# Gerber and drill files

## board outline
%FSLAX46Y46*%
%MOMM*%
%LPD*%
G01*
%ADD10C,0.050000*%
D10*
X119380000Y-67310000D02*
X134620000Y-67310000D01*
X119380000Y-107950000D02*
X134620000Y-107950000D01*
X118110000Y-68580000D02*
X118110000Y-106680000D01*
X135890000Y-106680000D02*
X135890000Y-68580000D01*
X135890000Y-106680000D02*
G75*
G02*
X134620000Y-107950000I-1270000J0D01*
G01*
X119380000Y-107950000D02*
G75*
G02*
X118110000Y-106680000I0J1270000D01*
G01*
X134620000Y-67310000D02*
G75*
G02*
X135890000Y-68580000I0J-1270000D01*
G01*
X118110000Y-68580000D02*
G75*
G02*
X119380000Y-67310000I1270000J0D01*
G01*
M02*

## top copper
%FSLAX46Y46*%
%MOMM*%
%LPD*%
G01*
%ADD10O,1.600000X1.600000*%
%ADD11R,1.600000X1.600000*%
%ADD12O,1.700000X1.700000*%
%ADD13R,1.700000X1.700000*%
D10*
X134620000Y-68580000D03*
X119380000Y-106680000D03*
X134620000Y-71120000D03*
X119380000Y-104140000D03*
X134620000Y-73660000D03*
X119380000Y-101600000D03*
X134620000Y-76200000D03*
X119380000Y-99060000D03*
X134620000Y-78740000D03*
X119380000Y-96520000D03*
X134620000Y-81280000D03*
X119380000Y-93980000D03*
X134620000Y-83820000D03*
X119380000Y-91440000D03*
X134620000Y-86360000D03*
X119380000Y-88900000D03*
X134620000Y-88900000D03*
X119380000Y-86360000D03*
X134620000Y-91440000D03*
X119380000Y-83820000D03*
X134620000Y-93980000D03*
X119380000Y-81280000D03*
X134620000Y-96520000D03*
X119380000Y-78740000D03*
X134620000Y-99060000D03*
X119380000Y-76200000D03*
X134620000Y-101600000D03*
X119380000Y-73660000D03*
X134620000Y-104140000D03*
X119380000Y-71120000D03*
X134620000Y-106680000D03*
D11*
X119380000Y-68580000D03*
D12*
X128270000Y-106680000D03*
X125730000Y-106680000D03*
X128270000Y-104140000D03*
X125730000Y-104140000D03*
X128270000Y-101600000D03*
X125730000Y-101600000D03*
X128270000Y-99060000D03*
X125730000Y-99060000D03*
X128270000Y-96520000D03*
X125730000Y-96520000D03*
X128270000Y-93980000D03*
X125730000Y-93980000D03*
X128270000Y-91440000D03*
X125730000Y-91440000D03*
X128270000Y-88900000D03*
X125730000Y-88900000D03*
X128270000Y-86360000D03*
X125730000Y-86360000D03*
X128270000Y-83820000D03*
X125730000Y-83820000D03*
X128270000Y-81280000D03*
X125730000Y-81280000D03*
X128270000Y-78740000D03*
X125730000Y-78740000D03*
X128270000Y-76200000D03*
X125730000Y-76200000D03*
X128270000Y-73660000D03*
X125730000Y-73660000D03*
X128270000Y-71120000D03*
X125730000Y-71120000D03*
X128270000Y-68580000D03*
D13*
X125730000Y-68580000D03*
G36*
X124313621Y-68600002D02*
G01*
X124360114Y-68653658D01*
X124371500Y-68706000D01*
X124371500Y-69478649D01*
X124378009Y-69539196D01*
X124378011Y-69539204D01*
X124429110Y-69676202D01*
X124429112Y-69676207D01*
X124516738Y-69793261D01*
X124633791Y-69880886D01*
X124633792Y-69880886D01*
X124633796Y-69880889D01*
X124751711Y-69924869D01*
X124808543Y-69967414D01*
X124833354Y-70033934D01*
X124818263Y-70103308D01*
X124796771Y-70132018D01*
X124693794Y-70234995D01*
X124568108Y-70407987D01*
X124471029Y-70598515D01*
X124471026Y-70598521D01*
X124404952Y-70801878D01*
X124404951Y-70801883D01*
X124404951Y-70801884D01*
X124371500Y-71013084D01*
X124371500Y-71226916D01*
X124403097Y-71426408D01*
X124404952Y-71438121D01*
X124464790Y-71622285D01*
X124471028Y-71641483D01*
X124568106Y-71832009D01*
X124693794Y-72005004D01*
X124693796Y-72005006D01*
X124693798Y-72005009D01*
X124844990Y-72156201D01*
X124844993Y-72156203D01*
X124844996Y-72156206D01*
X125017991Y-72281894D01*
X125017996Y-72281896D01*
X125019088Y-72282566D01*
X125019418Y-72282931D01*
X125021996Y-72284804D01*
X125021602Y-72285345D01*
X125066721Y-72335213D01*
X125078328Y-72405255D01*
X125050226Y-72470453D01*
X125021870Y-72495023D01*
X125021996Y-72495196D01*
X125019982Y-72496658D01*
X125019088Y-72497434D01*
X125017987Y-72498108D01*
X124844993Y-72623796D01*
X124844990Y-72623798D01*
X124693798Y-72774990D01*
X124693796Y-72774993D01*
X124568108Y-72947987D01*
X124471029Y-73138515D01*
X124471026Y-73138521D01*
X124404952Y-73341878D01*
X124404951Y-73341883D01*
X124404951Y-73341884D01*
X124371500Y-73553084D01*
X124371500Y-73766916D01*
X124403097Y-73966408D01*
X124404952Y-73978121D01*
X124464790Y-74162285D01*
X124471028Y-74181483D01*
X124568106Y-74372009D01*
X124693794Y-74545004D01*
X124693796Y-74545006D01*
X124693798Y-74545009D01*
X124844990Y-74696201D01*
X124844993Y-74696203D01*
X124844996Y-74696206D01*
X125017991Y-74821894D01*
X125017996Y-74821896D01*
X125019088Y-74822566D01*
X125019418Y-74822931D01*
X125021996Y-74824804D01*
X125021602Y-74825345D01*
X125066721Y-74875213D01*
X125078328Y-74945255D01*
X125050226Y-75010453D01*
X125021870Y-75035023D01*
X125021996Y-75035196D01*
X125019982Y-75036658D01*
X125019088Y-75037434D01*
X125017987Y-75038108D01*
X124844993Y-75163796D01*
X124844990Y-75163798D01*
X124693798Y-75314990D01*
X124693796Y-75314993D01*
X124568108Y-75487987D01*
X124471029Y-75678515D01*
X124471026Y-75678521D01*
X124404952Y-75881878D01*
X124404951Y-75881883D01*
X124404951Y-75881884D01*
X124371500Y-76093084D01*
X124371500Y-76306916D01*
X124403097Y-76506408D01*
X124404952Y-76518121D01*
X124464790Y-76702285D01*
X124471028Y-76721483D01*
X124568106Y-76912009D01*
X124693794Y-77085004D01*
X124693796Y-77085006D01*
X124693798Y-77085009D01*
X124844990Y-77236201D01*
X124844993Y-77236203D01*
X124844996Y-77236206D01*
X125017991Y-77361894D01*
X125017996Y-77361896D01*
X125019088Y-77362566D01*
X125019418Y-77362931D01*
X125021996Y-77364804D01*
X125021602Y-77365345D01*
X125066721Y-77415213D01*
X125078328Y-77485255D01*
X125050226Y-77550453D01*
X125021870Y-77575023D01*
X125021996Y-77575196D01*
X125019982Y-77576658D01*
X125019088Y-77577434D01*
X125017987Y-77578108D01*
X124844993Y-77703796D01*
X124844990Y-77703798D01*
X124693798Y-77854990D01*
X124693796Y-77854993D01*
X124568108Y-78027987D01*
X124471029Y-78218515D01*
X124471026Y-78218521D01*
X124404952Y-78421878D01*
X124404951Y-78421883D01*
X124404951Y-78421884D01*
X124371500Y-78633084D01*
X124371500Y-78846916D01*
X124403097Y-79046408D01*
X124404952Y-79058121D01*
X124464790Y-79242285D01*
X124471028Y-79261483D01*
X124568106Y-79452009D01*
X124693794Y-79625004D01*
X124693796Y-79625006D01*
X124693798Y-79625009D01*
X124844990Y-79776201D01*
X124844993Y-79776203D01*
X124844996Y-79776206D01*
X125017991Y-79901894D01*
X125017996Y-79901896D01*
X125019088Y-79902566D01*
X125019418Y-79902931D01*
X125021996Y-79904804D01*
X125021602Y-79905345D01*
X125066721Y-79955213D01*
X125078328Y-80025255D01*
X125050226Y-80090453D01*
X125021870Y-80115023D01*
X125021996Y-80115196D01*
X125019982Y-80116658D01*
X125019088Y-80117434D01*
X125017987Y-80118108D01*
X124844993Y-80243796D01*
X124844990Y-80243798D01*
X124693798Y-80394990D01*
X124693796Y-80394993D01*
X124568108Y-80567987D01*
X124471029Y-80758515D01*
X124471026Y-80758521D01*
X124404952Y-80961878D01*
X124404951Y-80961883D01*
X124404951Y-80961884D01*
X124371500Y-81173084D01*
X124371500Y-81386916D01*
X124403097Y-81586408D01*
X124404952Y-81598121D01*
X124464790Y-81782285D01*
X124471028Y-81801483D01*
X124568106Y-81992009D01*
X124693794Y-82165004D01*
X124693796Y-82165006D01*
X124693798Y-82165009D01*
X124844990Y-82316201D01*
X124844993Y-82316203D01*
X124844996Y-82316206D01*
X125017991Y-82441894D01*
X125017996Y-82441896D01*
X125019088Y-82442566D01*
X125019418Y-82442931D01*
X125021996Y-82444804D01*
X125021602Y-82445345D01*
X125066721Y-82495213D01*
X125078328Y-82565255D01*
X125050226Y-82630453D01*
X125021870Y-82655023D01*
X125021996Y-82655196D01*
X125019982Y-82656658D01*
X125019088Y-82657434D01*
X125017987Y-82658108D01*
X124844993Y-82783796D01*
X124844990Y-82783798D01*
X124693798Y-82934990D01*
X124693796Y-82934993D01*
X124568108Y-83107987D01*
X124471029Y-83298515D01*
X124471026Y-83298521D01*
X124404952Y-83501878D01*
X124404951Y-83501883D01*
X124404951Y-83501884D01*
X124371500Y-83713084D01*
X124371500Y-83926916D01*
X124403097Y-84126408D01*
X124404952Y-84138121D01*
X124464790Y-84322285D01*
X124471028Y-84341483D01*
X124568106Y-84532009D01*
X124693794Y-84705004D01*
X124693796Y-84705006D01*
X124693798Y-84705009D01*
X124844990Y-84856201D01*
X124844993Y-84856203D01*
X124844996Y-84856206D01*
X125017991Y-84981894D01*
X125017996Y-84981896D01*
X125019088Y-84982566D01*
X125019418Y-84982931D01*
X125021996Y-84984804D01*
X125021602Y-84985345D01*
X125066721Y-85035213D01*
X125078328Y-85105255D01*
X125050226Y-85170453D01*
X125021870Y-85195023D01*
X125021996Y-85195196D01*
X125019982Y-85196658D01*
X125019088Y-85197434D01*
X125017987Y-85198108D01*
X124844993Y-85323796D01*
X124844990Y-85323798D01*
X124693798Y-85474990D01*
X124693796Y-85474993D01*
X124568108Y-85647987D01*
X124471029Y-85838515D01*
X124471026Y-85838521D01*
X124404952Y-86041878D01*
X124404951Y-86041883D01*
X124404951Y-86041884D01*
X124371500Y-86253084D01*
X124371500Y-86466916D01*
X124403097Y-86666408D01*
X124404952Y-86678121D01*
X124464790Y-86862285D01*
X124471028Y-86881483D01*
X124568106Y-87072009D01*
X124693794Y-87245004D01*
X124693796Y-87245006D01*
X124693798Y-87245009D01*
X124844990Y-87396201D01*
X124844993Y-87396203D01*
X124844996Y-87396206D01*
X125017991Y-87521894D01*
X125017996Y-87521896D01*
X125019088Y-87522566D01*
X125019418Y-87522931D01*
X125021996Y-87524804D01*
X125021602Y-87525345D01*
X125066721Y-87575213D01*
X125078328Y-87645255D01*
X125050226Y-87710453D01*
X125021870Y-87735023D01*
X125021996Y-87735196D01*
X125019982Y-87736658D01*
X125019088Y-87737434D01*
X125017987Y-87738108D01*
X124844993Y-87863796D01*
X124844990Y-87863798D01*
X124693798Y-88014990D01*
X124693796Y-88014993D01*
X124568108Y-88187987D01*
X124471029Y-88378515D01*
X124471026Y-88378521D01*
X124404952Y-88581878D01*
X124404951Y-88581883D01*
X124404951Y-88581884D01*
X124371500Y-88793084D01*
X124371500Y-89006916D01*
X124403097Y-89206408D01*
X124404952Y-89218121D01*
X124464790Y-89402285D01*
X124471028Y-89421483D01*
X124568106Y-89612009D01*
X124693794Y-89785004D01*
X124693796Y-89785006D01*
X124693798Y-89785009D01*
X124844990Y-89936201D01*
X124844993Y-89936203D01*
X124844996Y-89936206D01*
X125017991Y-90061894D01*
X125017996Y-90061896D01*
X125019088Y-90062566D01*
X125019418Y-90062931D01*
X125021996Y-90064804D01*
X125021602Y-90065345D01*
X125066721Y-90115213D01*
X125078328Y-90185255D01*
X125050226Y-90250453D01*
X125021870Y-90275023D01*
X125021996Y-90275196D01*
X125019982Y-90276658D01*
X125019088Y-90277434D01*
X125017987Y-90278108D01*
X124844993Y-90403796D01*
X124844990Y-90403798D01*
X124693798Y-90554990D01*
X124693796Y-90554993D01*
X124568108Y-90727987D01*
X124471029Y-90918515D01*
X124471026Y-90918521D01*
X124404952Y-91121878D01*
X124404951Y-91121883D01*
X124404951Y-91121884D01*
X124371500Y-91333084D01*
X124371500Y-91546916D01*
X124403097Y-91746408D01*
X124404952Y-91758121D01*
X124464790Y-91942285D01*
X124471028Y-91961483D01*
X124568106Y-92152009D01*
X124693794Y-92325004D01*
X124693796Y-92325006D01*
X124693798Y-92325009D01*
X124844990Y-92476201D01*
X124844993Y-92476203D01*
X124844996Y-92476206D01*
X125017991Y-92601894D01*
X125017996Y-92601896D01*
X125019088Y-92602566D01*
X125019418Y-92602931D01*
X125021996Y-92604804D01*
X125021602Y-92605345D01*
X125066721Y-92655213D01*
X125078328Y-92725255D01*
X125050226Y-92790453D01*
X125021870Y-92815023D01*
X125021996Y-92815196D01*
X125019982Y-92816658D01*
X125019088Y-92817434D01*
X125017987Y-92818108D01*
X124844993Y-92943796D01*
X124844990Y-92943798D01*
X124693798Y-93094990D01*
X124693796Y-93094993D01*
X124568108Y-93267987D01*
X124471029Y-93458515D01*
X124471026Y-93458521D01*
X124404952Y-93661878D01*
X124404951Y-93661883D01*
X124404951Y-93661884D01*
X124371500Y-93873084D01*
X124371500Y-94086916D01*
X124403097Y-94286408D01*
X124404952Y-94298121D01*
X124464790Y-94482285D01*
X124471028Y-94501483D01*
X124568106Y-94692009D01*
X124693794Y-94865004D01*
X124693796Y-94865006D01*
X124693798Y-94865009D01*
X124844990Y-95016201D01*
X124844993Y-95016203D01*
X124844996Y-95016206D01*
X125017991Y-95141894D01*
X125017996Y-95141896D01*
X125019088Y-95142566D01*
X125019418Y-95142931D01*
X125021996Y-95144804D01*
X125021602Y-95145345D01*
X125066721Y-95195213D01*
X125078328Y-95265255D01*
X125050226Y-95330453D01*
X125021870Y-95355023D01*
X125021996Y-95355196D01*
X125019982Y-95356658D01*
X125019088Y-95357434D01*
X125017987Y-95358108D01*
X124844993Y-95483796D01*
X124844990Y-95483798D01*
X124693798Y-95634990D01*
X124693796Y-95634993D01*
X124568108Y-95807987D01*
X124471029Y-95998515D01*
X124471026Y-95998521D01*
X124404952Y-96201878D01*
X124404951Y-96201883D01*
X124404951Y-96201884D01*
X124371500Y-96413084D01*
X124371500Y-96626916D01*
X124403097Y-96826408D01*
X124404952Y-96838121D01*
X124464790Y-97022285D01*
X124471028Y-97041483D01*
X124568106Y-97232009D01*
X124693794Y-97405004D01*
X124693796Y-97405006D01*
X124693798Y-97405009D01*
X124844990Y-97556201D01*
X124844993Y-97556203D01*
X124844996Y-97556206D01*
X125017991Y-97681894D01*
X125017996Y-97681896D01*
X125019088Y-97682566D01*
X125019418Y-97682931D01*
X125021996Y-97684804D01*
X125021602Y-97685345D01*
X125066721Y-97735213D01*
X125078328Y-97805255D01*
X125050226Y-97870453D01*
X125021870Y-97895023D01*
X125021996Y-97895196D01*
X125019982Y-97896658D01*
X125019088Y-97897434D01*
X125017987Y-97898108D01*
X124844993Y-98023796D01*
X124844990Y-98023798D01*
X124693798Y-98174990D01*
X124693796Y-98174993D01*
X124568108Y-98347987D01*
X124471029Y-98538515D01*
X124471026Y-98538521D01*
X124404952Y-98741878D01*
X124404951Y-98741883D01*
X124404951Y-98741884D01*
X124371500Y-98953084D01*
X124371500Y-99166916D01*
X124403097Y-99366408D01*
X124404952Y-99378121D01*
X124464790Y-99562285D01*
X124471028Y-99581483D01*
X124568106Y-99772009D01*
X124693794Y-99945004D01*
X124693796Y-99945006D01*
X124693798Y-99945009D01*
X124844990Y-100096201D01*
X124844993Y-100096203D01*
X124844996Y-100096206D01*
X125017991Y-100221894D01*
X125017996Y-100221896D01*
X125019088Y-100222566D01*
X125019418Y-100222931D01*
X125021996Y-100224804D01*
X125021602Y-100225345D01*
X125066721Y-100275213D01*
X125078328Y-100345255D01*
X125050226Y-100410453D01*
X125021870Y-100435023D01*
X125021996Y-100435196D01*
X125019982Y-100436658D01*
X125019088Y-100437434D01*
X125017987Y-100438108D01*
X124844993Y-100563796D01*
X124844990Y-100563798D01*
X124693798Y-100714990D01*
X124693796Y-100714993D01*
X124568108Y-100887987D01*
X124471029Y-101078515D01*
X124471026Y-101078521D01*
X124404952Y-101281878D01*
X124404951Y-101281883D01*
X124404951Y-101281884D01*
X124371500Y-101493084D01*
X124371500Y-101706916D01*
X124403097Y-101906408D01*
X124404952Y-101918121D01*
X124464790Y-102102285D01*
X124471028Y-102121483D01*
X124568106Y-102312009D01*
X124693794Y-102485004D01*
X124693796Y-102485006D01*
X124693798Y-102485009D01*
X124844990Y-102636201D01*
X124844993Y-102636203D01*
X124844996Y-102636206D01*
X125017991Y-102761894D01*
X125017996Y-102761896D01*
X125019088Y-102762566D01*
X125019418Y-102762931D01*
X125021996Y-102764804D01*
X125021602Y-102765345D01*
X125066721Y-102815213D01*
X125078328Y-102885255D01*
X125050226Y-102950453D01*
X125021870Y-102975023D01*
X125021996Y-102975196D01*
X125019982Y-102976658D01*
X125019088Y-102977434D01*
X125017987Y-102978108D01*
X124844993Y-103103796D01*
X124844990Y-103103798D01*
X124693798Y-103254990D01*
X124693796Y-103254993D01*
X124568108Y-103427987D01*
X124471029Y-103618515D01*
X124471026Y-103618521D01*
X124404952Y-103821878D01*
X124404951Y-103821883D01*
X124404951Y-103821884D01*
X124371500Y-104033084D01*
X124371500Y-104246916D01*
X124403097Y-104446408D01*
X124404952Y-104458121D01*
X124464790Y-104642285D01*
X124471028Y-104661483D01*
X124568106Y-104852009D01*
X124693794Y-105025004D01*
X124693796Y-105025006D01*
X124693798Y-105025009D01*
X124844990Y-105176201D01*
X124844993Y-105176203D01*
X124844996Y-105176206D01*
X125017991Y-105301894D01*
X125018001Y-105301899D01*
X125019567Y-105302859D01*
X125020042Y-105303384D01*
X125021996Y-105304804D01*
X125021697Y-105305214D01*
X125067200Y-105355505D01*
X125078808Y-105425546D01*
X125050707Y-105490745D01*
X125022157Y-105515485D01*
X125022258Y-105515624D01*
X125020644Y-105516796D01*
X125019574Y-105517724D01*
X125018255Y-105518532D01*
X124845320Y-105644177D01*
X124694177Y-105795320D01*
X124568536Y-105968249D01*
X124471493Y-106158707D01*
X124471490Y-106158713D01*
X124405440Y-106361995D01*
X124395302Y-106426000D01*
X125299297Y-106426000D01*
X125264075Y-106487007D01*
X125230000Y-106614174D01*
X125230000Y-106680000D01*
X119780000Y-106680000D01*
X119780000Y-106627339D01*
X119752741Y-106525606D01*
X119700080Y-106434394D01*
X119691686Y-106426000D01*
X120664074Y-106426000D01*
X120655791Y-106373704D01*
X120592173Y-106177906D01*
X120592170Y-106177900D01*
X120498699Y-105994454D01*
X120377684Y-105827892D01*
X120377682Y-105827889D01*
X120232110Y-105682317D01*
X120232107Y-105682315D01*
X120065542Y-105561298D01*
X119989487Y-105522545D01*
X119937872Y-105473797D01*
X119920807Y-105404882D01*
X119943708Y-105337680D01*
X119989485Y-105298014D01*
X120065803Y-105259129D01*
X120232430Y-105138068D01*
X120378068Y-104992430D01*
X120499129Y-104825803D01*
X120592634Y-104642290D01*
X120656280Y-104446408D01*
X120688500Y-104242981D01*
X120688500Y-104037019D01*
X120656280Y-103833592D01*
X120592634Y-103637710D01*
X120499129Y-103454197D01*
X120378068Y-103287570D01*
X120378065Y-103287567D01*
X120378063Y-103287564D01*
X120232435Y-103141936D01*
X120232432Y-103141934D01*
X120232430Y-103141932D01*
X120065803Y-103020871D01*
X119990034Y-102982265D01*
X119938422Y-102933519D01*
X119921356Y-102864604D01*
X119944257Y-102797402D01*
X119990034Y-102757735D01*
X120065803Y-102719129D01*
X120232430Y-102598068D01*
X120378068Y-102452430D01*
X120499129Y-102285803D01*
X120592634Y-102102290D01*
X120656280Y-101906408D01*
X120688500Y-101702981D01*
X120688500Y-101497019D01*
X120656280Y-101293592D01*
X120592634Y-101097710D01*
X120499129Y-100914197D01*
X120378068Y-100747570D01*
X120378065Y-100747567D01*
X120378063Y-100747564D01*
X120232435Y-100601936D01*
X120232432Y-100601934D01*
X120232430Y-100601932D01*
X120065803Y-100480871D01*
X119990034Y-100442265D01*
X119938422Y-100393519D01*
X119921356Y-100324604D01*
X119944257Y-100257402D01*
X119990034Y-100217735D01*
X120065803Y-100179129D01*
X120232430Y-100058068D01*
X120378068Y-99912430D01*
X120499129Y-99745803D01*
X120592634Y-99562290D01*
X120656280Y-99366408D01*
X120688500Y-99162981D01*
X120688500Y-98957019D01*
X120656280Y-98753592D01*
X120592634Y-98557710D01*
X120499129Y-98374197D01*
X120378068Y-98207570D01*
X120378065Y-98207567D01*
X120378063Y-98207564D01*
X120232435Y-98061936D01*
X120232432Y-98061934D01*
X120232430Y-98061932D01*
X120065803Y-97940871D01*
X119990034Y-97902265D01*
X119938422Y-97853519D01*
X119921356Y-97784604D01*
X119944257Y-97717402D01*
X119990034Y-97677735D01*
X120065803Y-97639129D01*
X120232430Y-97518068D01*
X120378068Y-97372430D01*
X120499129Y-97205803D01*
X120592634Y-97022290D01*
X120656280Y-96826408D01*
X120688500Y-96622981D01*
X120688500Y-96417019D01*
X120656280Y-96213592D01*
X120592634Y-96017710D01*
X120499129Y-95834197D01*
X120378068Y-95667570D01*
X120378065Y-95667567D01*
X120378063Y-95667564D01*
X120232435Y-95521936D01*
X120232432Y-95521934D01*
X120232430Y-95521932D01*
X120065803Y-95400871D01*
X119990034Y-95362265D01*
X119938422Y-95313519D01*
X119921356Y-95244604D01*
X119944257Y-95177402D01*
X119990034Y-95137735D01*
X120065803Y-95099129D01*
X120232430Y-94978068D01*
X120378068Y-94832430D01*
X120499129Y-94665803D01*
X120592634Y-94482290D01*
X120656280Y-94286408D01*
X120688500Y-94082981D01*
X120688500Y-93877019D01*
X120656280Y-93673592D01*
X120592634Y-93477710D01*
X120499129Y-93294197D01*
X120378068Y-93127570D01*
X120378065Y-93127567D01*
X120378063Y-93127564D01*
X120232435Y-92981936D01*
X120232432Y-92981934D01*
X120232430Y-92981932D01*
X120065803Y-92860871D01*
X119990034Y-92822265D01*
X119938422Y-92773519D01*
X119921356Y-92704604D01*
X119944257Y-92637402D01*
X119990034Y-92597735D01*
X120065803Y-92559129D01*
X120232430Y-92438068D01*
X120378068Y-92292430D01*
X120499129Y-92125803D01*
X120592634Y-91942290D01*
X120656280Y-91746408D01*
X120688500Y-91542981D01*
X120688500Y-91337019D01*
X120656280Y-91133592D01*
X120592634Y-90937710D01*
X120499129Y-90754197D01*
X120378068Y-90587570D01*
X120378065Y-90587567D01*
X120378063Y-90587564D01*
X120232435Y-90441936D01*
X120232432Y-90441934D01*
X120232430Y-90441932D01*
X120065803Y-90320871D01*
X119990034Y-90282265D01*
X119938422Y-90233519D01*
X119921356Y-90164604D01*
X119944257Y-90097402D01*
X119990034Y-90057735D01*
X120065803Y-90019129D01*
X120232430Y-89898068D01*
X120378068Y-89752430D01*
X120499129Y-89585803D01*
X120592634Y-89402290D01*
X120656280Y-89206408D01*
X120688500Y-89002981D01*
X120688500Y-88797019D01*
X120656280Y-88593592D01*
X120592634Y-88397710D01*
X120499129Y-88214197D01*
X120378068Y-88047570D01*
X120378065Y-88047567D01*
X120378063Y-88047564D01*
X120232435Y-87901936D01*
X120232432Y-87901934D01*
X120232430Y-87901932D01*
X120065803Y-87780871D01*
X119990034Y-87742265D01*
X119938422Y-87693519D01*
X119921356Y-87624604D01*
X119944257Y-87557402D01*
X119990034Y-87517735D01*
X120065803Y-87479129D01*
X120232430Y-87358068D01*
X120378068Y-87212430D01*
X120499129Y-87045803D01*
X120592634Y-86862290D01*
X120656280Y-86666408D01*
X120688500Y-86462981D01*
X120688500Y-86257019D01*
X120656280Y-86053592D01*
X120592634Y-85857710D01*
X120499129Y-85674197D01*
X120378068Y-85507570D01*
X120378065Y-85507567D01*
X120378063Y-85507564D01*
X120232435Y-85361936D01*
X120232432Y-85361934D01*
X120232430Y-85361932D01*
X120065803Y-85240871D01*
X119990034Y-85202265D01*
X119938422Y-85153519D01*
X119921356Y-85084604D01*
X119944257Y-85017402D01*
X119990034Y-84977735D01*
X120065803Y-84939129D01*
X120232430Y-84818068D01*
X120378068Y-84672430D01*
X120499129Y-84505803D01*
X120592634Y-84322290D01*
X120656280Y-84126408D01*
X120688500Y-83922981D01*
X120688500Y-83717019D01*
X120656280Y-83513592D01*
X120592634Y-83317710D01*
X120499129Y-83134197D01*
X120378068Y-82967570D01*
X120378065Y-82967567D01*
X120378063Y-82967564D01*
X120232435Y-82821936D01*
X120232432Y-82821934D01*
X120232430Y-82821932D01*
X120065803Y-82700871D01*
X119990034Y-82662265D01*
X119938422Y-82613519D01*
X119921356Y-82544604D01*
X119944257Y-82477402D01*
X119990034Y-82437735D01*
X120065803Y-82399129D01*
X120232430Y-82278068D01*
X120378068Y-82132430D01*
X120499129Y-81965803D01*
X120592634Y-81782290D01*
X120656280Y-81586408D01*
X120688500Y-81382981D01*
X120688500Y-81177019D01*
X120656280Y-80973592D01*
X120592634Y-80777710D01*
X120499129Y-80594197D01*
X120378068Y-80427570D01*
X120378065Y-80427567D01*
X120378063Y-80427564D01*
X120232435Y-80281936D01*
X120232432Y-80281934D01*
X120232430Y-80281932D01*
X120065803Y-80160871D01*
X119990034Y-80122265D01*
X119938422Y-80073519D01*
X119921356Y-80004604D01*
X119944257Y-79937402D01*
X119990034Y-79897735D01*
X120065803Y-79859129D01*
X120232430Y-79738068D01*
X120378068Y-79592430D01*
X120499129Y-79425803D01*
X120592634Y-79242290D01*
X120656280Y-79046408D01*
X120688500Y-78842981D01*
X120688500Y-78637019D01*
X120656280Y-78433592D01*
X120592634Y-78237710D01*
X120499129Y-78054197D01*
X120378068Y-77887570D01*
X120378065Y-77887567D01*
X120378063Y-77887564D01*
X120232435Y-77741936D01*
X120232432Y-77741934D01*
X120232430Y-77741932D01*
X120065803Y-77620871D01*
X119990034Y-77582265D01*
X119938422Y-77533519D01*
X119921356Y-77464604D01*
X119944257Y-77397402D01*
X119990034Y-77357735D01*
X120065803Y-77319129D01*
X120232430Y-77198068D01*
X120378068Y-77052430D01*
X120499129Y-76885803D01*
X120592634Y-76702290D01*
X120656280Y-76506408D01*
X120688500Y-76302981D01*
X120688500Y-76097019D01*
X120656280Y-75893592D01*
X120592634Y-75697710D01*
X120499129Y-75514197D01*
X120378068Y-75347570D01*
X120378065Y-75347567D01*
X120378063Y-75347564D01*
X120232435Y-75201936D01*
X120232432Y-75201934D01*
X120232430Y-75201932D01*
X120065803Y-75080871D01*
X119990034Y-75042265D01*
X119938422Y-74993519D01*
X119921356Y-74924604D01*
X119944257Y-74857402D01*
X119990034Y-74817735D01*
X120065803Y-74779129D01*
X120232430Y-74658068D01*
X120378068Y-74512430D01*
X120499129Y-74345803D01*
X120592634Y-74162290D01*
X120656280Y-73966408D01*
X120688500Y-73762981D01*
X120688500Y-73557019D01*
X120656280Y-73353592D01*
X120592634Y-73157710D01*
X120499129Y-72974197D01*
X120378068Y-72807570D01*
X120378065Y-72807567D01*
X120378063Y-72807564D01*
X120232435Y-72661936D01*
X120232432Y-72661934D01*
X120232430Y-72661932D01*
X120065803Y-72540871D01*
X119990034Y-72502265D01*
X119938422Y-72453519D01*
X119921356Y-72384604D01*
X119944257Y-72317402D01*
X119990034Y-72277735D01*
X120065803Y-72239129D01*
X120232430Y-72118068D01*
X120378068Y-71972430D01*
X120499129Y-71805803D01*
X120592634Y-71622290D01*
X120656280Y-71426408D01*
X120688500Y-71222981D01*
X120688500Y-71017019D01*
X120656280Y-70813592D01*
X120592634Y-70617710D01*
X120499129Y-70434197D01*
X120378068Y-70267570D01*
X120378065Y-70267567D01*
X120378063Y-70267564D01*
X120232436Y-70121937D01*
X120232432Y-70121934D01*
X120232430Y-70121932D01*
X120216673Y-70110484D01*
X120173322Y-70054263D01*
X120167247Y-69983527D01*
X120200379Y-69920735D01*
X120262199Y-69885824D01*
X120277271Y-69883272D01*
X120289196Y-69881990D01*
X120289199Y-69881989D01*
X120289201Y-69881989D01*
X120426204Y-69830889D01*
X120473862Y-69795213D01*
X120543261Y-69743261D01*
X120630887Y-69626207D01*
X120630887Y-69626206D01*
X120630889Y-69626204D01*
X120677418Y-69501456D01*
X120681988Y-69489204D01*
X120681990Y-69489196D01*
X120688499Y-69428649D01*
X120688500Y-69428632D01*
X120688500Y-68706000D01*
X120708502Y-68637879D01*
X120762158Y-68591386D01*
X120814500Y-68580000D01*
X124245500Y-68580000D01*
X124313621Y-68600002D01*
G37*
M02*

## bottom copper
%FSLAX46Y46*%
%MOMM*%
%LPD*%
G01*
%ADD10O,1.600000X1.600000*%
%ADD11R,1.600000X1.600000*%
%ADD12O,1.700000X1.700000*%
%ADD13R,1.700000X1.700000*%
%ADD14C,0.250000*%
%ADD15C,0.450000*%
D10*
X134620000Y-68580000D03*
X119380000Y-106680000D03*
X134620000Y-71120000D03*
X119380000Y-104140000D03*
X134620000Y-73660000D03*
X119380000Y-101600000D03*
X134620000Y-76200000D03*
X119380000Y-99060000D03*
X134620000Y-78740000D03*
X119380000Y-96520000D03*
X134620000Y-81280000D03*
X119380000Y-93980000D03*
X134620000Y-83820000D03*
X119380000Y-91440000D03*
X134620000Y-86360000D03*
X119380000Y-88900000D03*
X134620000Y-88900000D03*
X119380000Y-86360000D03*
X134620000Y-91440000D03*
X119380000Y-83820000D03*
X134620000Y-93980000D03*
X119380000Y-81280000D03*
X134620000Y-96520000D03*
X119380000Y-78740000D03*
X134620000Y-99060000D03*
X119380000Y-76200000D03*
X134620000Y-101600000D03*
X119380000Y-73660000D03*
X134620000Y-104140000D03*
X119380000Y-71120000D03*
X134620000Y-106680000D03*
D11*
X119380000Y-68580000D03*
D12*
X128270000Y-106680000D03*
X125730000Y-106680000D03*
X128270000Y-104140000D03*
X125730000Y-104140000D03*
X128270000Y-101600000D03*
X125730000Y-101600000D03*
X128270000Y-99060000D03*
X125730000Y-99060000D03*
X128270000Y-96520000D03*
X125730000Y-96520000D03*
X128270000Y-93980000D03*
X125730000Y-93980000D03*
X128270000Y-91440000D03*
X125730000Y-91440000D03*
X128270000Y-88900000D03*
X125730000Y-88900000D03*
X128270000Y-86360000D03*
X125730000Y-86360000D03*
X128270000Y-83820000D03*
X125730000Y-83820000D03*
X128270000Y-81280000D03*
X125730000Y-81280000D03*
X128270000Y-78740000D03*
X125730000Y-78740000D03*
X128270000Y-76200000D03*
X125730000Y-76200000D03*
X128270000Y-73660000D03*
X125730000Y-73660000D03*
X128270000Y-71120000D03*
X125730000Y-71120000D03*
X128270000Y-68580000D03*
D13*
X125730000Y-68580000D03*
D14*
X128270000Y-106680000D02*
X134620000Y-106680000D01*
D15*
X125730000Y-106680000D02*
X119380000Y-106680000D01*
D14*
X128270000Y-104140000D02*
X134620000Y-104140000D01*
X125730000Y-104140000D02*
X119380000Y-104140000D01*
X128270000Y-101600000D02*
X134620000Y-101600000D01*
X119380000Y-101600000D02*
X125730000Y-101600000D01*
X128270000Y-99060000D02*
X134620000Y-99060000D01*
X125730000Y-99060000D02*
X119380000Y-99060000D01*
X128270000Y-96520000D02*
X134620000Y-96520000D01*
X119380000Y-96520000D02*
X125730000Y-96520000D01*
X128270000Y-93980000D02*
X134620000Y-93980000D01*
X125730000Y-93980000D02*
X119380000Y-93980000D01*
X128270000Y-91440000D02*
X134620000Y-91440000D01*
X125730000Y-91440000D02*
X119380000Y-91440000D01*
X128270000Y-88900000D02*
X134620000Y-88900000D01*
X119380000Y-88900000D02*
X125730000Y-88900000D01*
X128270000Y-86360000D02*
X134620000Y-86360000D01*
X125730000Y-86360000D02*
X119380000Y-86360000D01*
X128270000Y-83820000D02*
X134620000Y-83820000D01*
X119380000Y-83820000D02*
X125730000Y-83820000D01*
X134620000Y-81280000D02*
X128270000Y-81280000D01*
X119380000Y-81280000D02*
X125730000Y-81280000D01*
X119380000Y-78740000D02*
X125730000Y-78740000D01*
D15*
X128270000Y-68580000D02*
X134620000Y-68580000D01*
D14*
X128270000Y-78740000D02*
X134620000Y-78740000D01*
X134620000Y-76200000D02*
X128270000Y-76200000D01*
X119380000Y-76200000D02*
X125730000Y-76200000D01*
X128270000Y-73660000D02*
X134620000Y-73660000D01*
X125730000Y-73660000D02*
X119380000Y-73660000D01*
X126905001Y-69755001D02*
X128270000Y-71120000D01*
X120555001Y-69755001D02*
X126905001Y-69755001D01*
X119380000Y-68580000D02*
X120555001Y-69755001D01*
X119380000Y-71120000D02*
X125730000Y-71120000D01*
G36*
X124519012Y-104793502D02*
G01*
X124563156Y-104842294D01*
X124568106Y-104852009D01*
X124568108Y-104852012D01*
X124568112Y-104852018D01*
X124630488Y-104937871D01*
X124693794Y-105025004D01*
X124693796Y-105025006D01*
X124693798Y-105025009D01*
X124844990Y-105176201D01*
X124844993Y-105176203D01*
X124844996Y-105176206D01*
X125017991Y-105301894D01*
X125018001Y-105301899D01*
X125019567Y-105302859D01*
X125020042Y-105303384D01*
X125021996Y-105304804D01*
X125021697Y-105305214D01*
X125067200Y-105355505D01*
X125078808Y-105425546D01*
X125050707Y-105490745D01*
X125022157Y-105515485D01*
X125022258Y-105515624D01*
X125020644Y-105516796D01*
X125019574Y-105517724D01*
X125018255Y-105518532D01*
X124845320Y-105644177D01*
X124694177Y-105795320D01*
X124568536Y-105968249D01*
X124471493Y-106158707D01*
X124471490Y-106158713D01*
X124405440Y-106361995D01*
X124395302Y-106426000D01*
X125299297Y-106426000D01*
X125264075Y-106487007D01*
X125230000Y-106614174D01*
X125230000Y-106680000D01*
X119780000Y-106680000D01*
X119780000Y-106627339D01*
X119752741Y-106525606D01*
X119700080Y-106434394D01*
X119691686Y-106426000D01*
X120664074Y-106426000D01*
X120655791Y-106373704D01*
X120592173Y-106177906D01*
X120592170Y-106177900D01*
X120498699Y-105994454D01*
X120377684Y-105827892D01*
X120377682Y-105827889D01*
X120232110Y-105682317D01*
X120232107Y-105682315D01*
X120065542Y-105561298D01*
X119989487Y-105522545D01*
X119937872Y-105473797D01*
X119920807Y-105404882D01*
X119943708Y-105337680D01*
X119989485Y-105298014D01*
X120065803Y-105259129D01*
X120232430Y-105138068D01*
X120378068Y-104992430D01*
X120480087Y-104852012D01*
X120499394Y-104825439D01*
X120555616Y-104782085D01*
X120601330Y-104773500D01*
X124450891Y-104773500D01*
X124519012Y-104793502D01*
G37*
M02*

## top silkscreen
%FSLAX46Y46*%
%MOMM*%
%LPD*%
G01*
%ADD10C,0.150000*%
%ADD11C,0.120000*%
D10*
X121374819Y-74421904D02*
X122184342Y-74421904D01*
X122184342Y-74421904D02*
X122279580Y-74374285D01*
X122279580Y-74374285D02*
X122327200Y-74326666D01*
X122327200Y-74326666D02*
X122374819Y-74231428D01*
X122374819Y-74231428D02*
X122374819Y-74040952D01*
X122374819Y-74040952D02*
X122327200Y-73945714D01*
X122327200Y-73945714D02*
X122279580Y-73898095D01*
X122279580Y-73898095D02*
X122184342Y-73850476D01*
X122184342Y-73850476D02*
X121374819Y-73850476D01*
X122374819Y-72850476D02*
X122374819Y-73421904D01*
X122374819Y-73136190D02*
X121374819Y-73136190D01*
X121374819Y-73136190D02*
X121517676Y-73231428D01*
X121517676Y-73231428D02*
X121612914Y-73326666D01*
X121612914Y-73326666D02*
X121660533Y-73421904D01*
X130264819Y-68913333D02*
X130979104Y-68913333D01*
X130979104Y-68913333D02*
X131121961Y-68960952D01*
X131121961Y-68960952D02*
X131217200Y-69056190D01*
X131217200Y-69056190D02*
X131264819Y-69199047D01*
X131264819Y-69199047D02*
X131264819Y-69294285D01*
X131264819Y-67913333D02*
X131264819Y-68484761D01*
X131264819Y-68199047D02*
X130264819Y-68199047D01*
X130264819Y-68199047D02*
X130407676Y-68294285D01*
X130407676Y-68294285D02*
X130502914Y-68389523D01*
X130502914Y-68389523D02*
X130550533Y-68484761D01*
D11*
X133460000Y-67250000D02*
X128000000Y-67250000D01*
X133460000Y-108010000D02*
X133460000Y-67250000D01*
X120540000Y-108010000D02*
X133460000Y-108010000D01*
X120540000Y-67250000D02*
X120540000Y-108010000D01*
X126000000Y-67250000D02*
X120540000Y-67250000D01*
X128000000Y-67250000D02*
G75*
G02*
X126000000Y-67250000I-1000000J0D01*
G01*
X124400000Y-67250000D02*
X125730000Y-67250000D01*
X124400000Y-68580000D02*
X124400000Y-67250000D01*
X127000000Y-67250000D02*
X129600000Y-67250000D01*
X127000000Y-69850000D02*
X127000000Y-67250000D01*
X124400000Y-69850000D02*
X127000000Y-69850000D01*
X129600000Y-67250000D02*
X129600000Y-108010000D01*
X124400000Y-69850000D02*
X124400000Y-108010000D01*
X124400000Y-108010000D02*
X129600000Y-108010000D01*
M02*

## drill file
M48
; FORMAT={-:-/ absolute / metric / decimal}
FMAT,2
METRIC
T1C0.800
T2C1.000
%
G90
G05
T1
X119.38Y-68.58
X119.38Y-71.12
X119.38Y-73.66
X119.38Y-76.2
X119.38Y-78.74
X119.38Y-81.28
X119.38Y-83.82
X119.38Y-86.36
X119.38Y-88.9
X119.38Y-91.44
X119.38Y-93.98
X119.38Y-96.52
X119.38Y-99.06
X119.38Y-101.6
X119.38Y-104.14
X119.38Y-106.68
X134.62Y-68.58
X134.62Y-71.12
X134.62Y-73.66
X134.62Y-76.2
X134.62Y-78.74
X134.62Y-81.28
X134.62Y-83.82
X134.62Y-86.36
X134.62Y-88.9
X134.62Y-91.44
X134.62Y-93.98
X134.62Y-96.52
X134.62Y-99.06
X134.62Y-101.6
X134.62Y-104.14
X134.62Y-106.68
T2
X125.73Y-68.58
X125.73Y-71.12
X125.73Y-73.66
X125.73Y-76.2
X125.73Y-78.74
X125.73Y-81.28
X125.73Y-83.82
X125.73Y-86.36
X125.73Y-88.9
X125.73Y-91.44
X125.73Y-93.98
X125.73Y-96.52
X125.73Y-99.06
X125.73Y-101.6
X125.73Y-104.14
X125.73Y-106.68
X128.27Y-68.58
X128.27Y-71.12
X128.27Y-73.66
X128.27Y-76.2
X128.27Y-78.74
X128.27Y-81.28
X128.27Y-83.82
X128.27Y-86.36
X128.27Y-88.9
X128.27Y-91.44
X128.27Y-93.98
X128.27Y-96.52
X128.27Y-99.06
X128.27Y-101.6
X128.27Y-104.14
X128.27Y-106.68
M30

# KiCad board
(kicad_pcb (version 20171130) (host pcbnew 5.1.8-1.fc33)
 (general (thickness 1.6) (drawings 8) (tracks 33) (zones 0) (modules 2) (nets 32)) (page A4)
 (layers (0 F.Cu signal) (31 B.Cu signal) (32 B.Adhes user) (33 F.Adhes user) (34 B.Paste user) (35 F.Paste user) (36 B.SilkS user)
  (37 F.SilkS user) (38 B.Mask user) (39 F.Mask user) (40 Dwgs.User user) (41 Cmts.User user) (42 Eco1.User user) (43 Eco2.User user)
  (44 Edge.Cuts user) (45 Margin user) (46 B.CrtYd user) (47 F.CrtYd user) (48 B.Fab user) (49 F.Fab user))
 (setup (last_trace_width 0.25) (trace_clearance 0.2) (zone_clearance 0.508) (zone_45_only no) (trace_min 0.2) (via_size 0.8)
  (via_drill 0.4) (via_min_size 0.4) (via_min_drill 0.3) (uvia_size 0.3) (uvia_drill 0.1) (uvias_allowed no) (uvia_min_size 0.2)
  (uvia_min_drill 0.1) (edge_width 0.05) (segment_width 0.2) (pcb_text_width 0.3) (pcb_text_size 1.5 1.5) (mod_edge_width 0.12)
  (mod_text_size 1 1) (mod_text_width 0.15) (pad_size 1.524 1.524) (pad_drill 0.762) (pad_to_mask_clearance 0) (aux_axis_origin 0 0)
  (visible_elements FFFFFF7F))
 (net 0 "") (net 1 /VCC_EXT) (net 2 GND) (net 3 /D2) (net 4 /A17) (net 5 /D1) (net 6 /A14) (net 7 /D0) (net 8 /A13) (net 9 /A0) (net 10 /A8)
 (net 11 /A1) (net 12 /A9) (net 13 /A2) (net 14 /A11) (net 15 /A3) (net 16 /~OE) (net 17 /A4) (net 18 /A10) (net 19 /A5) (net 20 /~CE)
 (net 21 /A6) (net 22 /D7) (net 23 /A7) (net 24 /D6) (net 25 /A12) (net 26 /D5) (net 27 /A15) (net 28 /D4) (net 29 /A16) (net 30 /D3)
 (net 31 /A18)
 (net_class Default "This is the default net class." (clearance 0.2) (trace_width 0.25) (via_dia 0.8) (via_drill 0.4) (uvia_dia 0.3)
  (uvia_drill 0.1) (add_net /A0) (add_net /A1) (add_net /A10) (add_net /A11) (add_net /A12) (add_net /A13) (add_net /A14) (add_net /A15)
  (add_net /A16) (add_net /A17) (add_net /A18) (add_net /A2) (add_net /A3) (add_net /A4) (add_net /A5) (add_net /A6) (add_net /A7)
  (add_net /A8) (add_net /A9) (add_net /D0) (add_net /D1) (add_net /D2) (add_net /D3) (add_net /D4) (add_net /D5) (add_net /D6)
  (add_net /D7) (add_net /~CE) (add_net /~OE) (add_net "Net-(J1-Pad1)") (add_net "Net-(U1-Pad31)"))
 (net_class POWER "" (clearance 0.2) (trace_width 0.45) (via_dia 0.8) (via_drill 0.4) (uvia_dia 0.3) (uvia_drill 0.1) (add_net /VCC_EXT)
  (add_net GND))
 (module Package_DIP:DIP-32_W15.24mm (layer F.Cu) (at 119.38 68.58)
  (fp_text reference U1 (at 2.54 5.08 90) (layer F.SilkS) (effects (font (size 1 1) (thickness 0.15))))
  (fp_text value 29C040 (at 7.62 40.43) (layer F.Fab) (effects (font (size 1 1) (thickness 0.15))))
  (fp_line (start 14.08 -1.33) (end 8.62 -1.33) (layer F.SilkS) (width 0.12))
  (fp_line (start 14.08 39.43) (end 14.08 -1.33) (layer F.SilkS) (width 0.12))
  (fp_line (start 1.16 39.43) (end 14.08 39.43) (layer F.SilkS) (width 0.12))
  (fp_line (start 1.16 -1.33) (end 1.16 39.43) (layer F.SilkS) (width 0.12))
  (fp_line (start 6.62 -1.33) (end 1.16 -1.33) (layer F.SilkS) (width 0.12))
  (fp_arc (start 7.62 -1.33) (end 6.62 -1.33) (angle -180) (layer F.SilkS) (width 0.12))
  (pad 32 thru_hole oval (at 15.24 0) (size 1.6 1.6) (drill 0.8) (layers *.Cu *.Mask) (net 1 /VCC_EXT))
  (pad 16 thru_hole oval (at 0 38.1) (size 1.6 1.6) (drill 0.8) (layers *.Cu *.Mask) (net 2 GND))
  (pad 31 thru_hole oval (at 15.24 2.54) (size 1.6 1.6) (drill 0.8) (layers *.Cu *.Mask))
  (pad 15 thru_hole oval (at 0 35.56) (size 1.6 1.6) (drill 0.8) (layers *.Cu *.Mask) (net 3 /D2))
  (pad 30 thru_hole oval (at 15.24 5.08) (size 1.6 1.6) (drill 0.8) (layers *.Cu *.Mask) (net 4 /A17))
  (pad 14 thru_hole oval (at 0 33.02) (size 1.6 1.6) (drill 0.8) (layers *.Cu *.Mask) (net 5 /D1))
  (pad 29 thru_hole oval (at 15.24 7.62) (size 1.6 1.6) (drill 0.8) (layers *.Cu *.Mask) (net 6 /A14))
  (pad 13 thru_hole oval (at 0 30.48) (size 1.6 1.6) (drill 0.8) (layers *.Cu *.Mask) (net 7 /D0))
  (pad 28 thru_hole oval (at 15.24 10.16) (size 1.6 1.6) (drill 0.8) (layers *.Cu *.Mask) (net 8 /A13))
  (pad 12 thru_hole oval (at 0 27.94) (size 1.6 1.6) (drill 0.8) (layers *.Cu *.Mask) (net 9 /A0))
  (pad 27 thru_hole oval (at 15.24 12.7) (size 1.6 1.6) (drill 0.8) (layers *.Cu *.Mask) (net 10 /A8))
  (pad 11 thru_hole oval (at 0 25.4) (size 1.6 1.6) (drill 0.8) (layers *.Cu *.Mask) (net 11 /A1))
  (pad 26 thru_hole oval (at 15.24 15.24) (size 1.6 1.6) (drill 0.8) (layers *.Cu *.Mask) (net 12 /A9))
  (pad 10 thru_hole oval (at 0 22.86) (size 1.6 1.6) (drill 0.8) (layers *.Cu *.Mask) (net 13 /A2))
  (pad 25 thru_hole oval (at 15.24 17.78) (size 1.6 1.6) (drill 0.8) (layers *.Cu *.Mask) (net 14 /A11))
  (pad 9 thru_hole oval (at 0 20.32) (size 1.6 1.6) (drill 0.8) (layers *.Cu *.Mask) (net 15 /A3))
  (pad 24 thru_hole oval (at 15.24 20.32) (size 1.6 1.6) (drill 0.8) (layers *.Cu *.Mask) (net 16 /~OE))
  (pad 8 thru_hole oval (at 0 17.78) (size 1.6 1.6) (drill 0.8) (layers *.Cu *.Mask) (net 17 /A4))
  (pad 23 thru_hole oval (at 15.24 22.86) (size 1.6 1.6) (drill 0.8) (layers *.Cu *.Mask) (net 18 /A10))
  (pad 7 thru_hole oval (at 0 15.24) (size 1.6 1.6) (drill 0.8) (layers *.Cu *.Mask) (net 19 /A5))
  (pad 22 thru_hole oval (at 15.24 25.4) (size 1.6 1.6) (drill 0.8) (layers *.Cu *.Mask) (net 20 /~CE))
  (pad 6 thru_hole oval (at 0 12.7) (size 1.6 1.6) (drill 0.8) (layers *.Cu *.Mask) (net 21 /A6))
  (pad 21 thru_hole oval (at 15.24 27.94) (size 1.6 1.6) (drill 0.8) (layers *.Cu *.Mask) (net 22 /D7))
  (pad 5 thru_hole oval (at 0 10.16) (size 1.6 1.6) (drill 0.8) (layers *.Cu *.Mask) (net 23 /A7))
  (pad 20 thru_hole oval (at 15.24 30.48) (size 1.6 1.6) (drill 0.8) (layers *.Cu *.Mask) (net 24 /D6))
  (pad 4 thru_hole oval (at 0 7.62) (size 1.6 1.6) (drill 0.8) (layers *.Cu *.Mask) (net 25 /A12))
  (pad 19 thru_hole oval (at 15.24 33.02) (size 1.6 1.6) (drill 0.8) (layers *.Cu *.Mask) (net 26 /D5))
  (pad 3 thru_hole oval (at 0 5.08) (size 1.6 1.6) (drill 0.8) (layers *.Cu *.Mask) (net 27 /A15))
  (pad 18 thru_hole oval (at 15.24 35.56) (size 1.6 1.6) (drill 0.8) (layers *.Cu *.Mask) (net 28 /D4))
  (pad 2 thru_hole oval (at 0 2.54) (size 1.6 1.6) (drill 0.8) (layers *.Cu *.Mask) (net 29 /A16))
  (pad 17 thru_hole oval (at 15.24 38.1) (size 1.6 1.6) (drill 0.8) (layers *.Cu *.Mask) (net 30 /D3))
  (pad 1 thru_hole rect (at 0 0) (size 1.6 1.6) (drill 0.8) (layers *.Cu *.Mask) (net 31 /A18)))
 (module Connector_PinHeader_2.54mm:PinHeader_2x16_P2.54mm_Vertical (layer F.Cu) (at 125.73 68.58)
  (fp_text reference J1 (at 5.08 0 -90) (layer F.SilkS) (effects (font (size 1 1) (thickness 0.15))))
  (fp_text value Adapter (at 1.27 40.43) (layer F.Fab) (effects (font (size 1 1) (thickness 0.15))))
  (fp_line (start -1.33 -1.33) (end 0 -1.33) (layer F.SilkS) (width 0.12))
  (fp_line (start -1.33 0) (end -1.33 -1.33) (layer F.SilkS) (width 0.12))
  (fp_line (start 1.27 -1.33) (end 3.87 -1.33) (layer F.SilkS) (width 0.12))
  (fp_line (start 1.27 1.27) (end 1.27 -1.33) (layer F.SilkS) (width 0.12))
  (fp_line (start -1.33 1.27) (end 1.27 1.27) (layer F.SilkS) (width 0.12))
  (fp_line (start 3.87 -1.33) (end 3.87 39.43) (layer F.SilkS) (width 0.12))
  (fp_line (start -1.33 1.27) (end -1.33 39.43) (layer F.SilkS) (width 0.12))
  (fp_line (start -1.33 39.43) (end 3.87 39.43) (layer F.SilkS) (width 0.12))
  (pad 32 thru_hole oval (at 2.54 38.1) (size 1.7 1.7) (drill 1) (layers *.Cu *.Mask) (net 30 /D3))
  (pad 31 thru_hole oval (at 0 38.1) (size 1.7 1.7) (drill 1) (layers *.Cu *.Mask) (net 2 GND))
  (pad 30 thru_hole oval (at 2.54 35.56) (size 1.7 1.7) (drill 1) (layers *.Cu *.Mask) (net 28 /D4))
  (pad 29 thru_hole oval (at 0 35.56) (size 1.7 1.7) (drill 1) (layers *.Cu *.Mask) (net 3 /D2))
  (pad 28 thru_hole oval (at 2.54 33.02) (size 1.7 1.7) (drill 1) (layers *.Cu *.Mask) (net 26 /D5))
  (pad 27 thru_hole oval (at 0 33.02) (size 1.7 1.7) (drill 1) (layers *.Cu *.Mask) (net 5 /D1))
  (pad 26 thru_hole oval (at 2.54 30.48) (size 1.7 1.7) (drill 1) (layers *.Cu *.Mask) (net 24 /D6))
  (pad 25 thru_hole oval (at 0 30.48) (size 1.7 1.7) (drill 1) (layers *.Cu *.Mask) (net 7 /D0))
  (pad 24 thru_hole oval (at 2.54 27.94) (size 1.7 1.7) (drill 1) (layers *.Cu *.Mask) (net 22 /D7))
  (pad 23 thru_hole oval (at 0 27.94) (size 1.7 1.7) (drill 1) (layers *.Cu *.Mask) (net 9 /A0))
  (pad 22 thru_hole oval (at 2.54 25.4) (size 1.7 1.7) (drill 1) (layers *.Cu *.Mask) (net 20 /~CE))
  (pad 21 thru_hole oval (at 0 25.4) (size 1.7 1.7) (drill 1) (layers *.Cu *.Mask) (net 11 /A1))
  (pad 20 thru_hole oval (at 2.54 22.86) (size 1.7 1.7) (drill 1) (layers *.Cu *.Mask) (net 18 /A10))
  (pad 19 thru_hole oval (at 0 22.86) (size 1.7 1.7) (drill 1) (layers *.Cu *.Mask) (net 13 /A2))
  (pad 18 thru_hole oval (at 2.54 20.32) (size 1.7 1.7) (drill 1) (layers *.Cu *.Mask) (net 16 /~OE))
  (pad 17 thru_hole oval (at 0 20.32) (size 1.7 1.7) (drill 1) (layers *.Cu *.Mask) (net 15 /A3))
  (pad 16 thru_hole oval (at 2.54 17.78) (size 1.7 1.7) (drill 1) (layers *.Cu *.Mask) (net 14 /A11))
  (pad 15 thru_hole oval (at 0 17.78) (size 1.7 1.7) (drill 1) (layers *.Cu *.Mask) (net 17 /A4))
  (pad 14 thru_hole oval (at 2.54 15.24) (size 1.7 1.7) (drill 1) (layers *.Cu *.Mask) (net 12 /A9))
  (pad 13 thru_hole oval (at 0 15.24) (size 1.7 1.7) (drill 1) (layers *.Cu *.Mask) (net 19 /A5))
  (pad 12 thru_hole oval (at 2.54 12.7) (size 1.7 1.7) (drill 1) (layers *.Cu *.Mask) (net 10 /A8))
  (pad 11 thru_hole oval (at 0 12.7) (size 1.7 1.7) (drill 1) (layers *.Cu *.Mask) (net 21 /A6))
  (pad 10 thru_hole oval (at 2.54 10.16) (size 1.7 1.7) (drill 1) (layers *.Cu *.Mask) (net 8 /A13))
  (pad 9 thru_hole oval (at 0 10.16) (size 1.7 1.7) (drill 1) (layers *.Cu *.Mask) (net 23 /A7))
  (pad 8 thru_hole oval (at 2.54 7.62) (size 1.7 1.7) (drill 1) (layers *.Cu *.Mask) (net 6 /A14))
  (pad 7 thru_hole oval (at 0 7.62) (size 1.7 1.7) (drill 1) (layers *.Cu *.Mask) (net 25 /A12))
  (pad 6 thru_hole oval (at 2.54 5.08) (size 1.7 1.7) (drill 1) (layers *.Cu *.Mask) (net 4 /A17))
  (pad 5 thru_hole oval (at 0 5.08) (size 1.7 1.7) (drill 1) (layers *.Cu *.Mask) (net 27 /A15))
  (pad 4 thru_hole oval (at 2.54 2.54) (size 1.7 1.7) (drill 1) (layers *.Cu *.Mask) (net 31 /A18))
  (pad 3 thru_hole oval (at 0 2.54) (size 1.7 1.7) (drill 1) (layers *.Cu *.Mask) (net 29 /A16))
  (pad 2 thru_hole oval (at 2.54 0) (size 1.7 1.7) (drill 1) (layers *.Cu *.Mask) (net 1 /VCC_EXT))
  (pad 1 thru_hole rect (at 0 0) (size 1.7 1.7) (drill 1) (layers *.Cu *.Mask)))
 (gr_line (start 119.38 67.31) (end 134.62 67.31) (layer Edge.Cuts) (width 0.05))
 (gr_line (start 119.38 107.95) (end 134.62 107.95) (layer Edge.Cuts) (width 0.05))
 (gr_line (start 118.11 68.58) (end 118.11 106.68) (layer Edge.Cuts) (width 0.05))
 (gr_line (start 135.89 106.68) (end 135.89 68.58) (layer Edge.Cuts) (width 0.05))
 (gr_arc (start 134.62 106.68) (end 134.62 107.95) (angle -90) (layer Edge.Cuts) (width 0.05))
 (gr_arc (start 119.38 106.68) (end 118.11 106.68) (angle -90) (layer Edge.Cuts) (width 0.05))
 (gr_arc (start 134.62 68.58) (end 135.89 68.58) (angle -90) (layer Edge.Cuts) (width 0.05))
 (gr_arc (start 119.38 68.58) (end 119.38 67.31) (angle -90) (layer Edge.Cuts) (width 0.05))
 (segment (start 128.27 106.68) (end 134.62 106.68) (width 0.25) (layer B.Cu) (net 30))
 (segment (start 125.73 106.68) (end 119.38 106.68) (width 0.45) (layer B.Cu) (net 2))
 (segment (start 128.27 104.14) (end 134.62 104.14) (width 0.25) (layer B.Cu) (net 28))
 (segment (start 125.73 104.14) (end 119.38 104.14) (width 0.25) (layer B.Cu) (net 3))
 (segment (start 128.27 101.6) (end 134.62 101.6) (width 0.25) (layer B.Cu) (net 26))
 (segment (start 119.38 101.6) (end 125.73 101.6) (width 0.25) (layer B.Cu) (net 5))
 (segment (start 128.27 99.06) (end 134.62 99.06) (width 0.25) (layer B.Cu) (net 24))
 (segment (start 125.73 99.06) (end 119.38 99.06) (width 0.25) (layer B.Cu) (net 7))
 (segment (start 128.27 96.52) (end 134.62 96.52) (width 0.25) (layer B.Cu) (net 22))
 (segment (start 119.38 96.52) (end 125.73 96.52) (width 0.25) (layer B.Cu) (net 9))
 (segment (start 128.27 93.98) (end 134.62 93.98) (width 0.25) (layer B.Cu) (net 20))
 (segment (start 125.73 93.98) (end 119.38 93.98) (width 0.25) (layer B.Cu) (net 11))
 (segment (start 128.27 91.44) (end 134.62 91.44) (width 0.25) (layer B.Cu) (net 18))
 (segment (start 125.73 91.44) (end 119.38 91.44) (width 0.25) (layer B.Cu) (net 13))
 (segment (start 128.27 88.9) (end 134.62 88.9) (width 0.25) (layer B.Cu) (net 16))
 (segment (start 119.38 88.9) (end 125.73 88.9) (width 0.25) (layer B.Cu) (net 15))
 (segment (start 128.27 86.36) (end 134.62 86.36) (width 0.25) (layer B.Cu) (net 14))
 (segment (start 125.73 86.36) (end 119.38 86.36) (width 0.25) (layer B.Cu) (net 17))
 (segment (start 128.27 83.82) (end 134.62 83.82) (width 0.25) (layer B.Cu) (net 12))
 (segment (start 119.38 83.82) (end 125.73 83.82) (width 0.25) (layer B.Cu) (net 19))
 (segment (start 134.62 81.28) (end 128.27 81.28) (width 0.25) (layer B.Cu) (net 10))
 (segment (start 119.38 81.28) (end 125.73 81.28) (width 0.25) (layer B.Cu) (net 21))
 (segment (start 119.38 78.74) (end 125.73 78.74) (width 0.25) (layer B.Cu) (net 23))
 (segment (start 128.27 68.58) (end 134.62 68.58) (width 0.45) (layer B.Cu) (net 1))
 (segment (start 128.27 78.74) (end 134.62 78.74) (width 0.25) (layer B.Cu) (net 8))
 (segment (start 134.62 76.2) (end 128.27 76.2) (width 0.25) (layer B.Cu) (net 6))
 (segment (start 119.38 76.2) (end 125.73 76.2) (width 0.25) (layer B.Cu) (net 25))
 (segment (start 128.27 73.66) (end 134.62 73.66) (width 0.25) (layer B.Cu) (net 4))
 (segment (start 125.73 73.66) (end 119.38 73.66) (width 0.25) (layer B.Cu) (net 27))
 (segment (start 126.905001 69.755001) (end 128.27 71.12) (width 0.25) (layer B.Cu) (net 31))
 (segment (start 120.555001 69.755001) (end 126.905001 69.755001) (width 0.25) (layer B.Cu) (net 31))
 (segment (start 119.38 68.58) (end 120.555001 69.755001) (width 0.25) (layer B.Cu) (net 31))
 (segment (start 119.38 71.12) (end 125.73 71.12) (width 0.25) (layer B.Cu) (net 29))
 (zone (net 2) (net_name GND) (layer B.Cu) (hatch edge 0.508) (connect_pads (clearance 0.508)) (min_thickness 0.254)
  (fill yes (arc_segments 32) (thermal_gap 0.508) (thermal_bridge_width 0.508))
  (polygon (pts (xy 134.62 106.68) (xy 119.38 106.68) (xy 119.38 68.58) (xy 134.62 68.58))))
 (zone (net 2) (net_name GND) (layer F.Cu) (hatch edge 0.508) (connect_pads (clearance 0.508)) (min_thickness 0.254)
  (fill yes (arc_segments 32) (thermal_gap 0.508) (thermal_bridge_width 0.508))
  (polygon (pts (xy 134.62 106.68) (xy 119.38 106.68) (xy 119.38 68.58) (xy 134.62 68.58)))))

